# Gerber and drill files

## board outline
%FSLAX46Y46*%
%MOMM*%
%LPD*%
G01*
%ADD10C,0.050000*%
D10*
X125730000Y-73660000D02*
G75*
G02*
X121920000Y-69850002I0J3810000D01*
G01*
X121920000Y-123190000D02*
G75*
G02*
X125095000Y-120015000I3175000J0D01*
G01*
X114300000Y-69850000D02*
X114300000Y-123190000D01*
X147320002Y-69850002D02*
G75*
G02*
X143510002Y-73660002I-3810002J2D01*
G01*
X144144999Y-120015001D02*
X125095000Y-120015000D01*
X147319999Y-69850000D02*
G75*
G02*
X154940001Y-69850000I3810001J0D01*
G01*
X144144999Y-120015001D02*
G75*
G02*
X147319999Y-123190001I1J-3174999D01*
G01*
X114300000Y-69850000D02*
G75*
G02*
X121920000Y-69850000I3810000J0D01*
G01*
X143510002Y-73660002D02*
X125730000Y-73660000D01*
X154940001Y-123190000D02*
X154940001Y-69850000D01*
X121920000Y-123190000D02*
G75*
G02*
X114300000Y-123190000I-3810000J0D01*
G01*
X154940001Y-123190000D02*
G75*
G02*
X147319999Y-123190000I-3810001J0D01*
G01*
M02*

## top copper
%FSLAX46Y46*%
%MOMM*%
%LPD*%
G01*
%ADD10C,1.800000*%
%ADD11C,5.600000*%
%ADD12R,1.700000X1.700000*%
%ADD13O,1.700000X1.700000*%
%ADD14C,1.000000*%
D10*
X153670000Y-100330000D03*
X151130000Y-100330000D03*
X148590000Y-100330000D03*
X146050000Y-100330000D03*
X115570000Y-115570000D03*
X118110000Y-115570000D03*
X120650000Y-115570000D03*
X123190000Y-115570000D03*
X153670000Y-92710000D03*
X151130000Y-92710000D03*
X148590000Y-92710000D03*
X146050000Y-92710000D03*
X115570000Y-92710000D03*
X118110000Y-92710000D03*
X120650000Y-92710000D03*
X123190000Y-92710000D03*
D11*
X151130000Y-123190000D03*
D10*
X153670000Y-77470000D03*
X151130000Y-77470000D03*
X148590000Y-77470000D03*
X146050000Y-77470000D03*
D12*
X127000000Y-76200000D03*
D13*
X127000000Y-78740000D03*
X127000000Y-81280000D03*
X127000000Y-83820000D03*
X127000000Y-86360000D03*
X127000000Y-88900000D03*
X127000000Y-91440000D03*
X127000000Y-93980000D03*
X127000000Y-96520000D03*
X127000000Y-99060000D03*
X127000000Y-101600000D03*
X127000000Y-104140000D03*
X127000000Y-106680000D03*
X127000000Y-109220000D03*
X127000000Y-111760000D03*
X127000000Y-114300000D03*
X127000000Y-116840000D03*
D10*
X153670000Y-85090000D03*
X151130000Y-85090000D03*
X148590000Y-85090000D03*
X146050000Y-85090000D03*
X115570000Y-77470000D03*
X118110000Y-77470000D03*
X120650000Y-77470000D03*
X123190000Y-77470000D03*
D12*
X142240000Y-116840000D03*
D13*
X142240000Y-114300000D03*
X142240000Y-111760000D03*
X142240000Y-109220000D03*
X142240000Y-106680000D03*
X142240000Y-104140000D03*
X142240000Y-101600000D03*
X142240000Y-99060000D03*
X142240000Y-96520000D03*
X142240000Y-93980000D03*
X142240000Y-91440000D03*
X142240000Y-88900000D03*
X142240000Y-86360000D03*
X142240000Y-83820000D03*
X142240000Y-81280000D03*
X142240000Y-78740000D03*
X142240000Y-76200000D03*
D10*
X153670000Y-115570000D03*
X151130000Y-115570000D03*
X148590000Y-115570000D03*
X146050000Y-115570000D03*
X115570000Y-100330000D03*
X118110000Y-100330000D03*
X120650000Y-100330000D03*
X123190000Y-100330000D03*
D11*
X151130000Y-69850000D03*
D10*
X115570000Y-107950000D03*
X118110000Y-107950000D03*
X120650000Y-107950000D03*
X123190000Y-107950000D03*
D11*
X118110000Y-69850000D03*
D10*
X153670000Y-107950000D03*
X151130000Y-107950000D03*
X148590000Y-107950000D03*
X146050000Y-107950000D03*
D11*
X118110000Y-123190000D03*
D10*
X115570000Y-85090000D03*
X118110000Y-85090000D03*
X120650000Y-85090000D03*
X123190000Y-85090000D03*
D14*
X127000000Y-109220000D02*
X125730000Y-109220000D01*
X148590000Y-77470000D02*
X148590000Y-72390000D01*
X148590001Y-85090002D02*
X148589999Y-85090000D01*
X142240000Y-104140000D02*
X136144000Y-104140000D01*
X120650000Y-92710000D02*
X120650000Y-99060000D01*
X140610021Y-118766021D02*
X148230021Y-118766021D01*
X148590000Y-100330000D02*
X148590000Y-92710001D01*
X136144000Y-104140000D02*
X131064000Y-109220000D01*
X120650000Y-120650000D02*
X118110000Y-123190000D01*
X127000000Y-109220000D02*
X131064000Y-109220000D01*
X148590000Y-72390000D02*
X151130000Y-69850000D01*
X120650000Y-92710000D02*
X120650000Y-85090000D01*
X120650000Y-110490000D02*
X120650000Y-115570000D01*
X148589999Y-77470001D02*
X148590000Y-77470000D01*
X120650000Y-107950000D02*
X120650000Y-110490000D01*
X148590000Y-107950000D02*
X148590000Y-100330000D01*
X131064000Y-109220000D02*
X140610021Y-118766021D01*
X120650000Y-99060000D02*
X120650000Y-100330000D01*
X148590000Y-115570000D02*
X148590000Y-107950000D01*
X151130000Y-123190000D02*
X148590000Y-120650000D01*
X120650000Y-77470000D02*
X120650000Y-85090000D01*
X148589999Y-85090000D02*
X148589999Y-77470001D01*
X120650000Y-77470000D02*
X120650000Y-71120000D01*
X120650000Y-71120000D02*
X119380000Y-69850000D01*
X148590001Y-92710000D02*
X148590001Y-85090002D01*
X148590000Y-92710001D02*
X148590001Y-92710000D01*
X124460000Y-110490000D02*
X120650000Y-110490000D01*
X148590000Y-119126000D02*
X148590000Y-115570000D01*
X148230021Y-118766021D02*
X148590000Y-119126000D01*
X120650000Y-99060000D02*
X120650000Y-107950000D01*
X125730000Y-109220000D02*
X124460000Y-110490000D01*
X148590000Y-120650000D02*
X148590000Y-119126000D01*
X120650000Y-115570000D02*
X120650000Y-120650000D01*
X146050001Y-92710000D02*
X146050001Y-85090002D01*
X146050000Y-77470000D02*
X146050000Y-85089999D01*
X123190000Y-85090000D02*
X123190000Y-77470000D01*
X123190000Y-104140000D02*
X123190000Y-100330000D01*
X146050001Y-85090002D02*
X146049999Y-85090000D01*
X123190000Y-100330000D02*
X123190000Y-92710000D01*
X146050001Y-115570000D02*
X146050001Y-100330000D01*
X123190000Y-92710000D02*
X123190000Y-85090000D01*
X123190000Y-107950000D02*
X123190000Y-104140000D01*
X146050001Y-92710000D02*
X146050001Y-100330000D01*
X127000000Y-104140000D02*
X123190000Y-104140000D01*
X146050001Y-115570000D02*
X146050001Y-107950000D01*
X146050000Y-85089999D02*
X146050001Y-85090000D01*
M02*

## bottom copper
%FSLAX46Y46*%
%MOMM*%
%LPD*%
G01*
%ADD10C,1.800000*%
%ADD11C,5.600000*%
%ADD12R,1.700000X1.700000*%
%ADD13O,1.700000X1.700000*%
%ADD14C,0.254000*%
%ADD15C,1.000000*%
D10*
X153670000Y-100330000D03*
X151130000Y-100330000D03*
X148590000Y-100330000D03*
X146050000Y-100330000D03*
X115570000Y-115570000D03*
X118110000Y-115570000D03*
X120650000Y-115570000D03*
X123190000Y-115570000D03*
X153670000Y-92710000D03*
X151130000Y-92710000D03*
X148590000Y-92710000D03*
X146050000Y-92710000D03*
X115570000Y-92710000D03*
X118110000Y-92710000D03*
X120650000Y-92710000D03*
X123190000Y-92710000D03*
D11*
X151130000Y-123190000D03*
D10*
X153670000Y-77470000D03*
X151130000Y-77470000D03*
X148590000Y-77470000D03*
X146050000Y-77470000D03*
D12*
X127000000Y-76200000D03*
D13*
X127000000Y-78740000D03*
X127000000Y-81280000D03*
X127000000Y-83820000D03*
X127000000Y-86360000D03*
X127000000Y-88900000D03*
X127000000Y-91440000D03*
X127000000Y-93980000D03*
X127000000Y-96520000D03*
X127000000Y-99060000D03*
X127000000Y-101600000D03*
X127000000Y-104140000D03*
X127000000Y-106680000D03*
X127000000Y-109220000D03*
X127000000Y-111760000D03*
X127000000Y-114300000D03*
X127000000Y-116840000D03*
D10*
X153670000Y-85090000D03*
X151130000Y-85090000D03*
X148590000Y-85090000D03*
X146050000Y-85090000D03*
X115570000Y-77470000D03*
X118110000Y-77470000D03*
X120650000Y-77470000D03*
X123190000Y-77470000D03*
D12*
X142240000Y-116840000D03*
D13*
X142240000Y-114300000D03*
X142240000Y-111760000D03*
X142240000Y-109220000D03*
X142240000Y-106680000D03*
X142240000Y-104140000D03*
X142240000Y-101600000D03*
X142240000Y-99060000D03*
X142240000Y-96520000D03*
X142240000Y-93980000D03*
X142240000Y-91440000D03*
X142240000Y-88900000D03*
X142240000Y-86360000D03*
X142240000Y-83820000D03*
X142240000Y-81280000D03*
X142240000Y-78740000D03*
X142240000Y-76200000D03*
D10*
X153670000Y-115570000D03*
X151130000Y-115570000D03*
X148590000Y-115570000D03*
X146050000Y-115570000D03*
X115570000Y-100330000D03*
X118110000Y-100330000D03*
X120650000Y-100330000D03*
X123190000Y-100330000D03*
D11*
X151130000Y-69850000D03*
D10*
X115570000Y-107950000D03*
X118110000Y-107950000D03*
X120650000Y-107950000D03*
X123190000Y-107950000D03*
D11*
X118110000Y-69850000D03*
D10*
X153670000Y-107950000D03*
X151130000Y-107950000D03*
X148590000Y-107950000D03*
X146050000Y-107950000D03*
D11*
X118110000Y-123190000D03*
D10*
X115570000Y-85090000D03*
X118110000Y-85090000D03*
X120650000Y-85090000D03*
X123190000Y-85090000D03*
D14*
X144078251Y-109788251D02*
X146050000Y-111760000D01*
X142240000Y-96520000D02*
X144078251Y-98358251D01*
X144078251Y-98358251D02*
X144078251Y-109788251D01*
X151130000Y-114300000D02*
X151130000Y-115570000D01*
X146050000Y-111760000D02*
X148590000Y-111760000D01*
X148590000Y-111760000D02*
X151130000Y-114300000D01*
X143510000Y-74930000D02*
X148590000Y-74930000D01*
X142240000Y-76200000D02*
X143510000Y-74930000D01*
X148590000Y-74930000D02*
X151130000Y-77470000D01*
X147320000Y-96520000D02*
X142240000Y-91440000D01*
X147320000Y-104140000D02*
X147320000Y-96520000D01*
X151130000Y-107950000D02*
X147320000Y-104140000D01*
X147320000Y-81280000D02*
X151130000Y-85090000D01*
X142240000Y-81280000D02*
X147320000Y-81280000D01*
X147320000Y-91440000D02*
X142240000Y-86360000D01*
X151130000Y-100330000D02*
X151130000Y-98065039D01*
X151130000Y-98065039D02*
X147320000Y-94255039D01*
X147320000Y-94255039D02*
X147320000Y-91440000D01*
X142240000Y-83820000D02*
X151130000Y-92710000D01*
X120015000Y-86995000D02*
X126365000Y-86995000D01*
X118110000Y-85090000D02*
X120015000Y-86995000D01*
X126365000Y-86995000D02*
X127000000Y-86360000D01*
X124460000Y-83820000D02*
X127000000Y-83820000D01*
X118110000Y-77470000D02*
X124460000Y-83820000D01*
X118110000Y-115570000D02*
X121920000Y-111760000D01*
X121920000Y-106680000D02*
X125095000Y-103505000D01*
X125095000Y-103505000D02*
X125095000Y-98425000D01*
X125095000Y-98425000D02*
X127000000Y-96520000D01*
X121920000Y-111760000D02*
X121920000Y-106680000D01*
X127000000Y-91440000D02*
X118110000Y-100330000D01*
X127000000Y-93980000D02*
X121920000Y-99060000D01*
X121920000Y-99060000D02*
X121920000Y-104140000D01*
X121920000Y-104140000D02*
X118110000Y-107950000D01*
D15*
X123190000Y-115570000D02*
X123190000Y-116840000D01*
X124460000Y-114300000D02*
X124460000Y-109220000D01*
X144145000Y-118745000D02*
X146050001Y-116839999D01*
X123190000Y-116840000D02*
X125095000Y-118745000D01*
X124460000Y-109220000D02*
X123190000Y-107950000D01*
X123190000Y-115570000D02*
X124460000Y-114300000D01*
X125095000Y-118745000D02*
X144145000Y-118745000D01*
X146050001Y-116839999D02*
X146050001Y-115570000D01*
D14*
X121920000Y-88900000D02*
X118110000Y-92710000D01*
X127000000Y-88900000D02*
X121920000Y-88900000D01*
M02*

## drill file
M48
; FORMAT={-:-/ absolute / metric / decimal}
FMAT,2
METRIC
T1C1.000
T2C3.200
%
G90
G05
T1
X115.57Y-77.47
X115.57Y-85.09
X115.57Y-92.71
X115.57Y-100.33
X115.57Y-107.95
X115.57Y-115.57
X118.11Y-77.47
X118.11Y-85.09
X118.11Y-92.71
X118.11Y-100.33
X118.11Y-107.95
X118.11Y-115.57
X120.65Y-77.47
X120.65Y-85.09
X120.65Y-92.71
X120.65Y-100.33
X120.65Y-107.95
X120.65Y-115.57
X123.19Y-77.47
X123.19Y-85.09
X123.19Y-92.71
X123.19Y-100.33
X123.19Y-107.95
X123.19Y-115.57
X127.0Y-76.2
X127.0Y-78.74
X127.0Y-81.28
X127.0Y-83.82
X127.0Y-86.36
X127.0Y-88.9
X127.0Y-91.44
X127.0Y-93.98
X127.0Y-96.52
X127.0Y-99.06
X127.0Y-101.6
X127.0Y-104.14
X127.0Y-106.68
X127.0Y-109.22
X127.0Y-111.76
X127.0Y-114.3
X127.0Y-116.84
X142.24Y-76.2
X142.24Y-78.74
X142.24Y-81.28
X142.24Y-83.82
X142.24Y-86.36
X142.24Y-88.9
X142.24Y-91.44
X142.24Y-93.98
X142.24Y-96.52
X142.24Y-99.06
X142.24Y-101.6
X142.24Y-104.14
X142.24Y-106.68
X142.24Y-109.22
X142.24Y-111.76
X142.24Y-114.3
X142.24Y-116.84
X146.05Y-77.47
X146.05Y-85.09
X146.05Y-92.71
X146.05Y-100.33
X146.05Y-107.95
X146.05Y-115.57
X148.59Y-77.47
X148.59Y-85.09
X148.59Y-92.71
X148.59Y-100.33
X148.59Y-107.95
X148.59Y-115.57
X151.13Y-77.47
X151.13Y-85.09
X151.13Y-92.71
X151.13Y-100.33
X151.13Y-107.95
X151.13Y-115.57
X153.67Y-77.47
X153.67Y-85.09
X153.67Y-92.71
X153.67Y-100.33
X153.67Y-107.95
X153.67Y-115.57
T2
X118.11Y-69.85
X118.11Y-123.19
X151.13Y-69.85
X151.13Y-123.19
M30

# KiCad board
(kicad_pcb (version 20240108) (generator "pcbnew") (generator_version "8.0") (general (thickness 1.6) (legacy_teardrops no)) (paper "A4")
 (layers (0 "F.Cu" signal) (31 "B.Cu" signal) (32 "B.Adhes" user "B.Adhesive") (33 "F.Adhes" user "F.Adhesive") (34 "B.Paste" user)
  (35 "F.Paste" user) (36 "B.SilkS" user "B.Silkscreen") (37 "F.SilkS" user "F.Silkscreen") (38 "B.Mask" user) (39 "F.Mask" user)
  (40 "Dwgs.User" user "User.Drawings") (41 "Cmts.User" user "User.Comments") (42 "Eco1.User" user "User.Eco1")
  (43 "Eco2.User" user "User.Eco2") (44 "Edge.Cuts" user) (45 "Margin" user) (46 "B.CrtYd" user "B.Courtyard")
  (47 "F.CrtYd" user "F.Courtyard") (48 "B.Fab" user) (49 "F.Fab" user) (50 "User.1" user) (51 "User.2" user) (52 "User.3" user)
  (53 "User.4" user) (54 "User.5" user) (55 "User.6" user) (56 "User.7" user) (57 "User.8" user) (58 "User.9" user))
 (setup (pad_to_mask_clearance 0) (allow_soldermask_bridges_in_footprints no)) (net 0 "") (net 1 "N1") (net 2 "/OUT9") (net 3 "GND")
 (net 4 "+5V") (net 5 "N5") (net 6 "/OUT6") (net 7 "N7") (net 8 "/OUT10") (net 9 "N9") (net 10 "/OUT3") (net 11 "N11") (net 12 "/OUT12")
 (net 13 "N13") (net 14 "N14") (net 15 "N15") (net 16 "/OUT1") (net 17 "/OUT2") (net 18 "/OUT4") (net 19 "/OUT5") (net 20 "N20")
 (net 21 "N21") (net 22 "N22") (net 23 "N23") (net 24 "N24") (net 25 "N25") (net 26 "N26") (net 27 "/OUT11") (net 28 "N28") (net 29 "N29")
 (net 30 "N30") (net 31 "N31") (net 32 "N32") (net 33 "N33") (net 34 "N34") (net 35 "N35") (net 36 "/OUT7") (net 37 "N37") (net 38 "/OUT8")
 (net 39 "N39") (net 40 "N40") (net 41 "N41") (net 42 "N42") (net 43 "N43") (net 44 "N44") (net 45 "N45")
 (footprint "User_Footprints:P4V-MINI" (layer "F.Cu") (at 153.67 100.33 180)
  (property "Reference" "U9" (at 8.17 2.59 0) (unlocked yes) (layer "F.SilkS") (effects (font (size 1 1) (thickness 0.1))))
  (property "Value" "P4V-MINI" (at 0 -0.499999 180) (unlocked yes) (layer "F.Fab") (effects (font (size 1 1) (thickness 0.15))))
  (pad "1" thru_hole circle (at 0 0 180) (size 1.8 1.8) (drill 1) (layers "*.Cu" "*.Mask") (remove_unused_layers no) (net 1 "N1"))
  (pad "2" thru_hole circle (at 2.54 0 180) (size 1.8 1.8) (drill 1) (layers "*.Cu" "*.Mask") (remove_unused_layers no) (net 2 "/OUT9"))
  (pad "3" thru_hole circle (at 5.08 0 180) (size 1.8 1.8) (drill 1) (layers "*.Cu" "*.Mask") (remove_unused_layers no) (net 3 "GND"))
  (pad "4" thru_hole circle (at 7.62 0 180) (size 1.8 1.8) (drill 1) (layers "*.Cu" "*.Mask") (remove_unused_layers no) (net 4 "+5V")))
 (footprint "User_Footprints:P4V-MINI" (layer "F.Cu") (at 115.57 115.57)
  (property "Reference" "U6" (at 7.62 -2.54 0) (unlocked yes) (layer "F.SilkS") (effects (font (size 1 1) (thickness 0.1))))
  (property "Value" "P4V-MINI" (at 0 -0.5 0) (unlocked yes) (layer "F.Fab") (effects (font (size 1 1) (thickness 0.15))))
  (pad "1" thru_hole circle (at 0 0) (size 1.8 1.8) (drill 1) (layers "*.Cu" "*.Mask") (remove_unused_layers no) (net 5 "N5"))
  (pad "2" thru_hole circle (at 2.54 0) (size 1.8 1.8) (drill 1) (layers "*.Cu" "*.Mask") (remove_unused_layers no) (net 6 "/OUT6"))
  (pad "3" thru_hole circle (at 5.08 0) (size 1.8 1.8) (drill 1) (layers "*.Cu" "*.Mask") (remove_unused_layers no) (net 3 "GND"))
  (pad "4" thru_hole circle (at 7.62 0) (size 1.8 1.8) (drill 1) (layers "*.Cu" "*.Mask") (remove_unused_layers no) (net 4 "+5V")))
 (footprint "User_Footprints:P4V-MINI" (layer "F.Cu") (at 153.67 92.71 180)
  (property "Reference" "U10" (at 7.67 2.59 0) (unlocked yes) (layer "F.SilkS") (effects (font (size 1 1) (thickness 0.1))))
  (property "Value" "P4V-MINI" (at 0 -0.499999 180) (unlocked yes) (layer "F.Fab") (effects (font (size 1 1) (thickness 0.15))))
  (pad "1" thru_hole circle (at 0 0 180) (size 1.8 1.8) (drill 1) (layers "*.Cu" "*.Mask") (remove_unused_layers no) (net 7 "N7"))
  (pad "2" thru_hole circle (at 2.54 0 180) (size 1.8 1.8) (drill 1) (layers "*.Cu" "*.Mask") (remove_unused_layers no) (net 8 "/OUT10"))
  (pad "3" thru_hole circle (at 5.08 0 180) (size 1.8 1.8) (drill 1) (layers "*.Cu" "*.Mask") (remove_unused_layers no) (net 3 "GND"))
  (pad "4" thru_hole circle (at 7.62 0 180) (size 1.8 1.8) (drill 1) (layers "*.Cu" "*.Mask") (remove_unused_layers no) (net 4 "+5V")))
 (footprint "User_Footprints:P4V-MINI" (layer "F.Cu") (at 115.57 92.71)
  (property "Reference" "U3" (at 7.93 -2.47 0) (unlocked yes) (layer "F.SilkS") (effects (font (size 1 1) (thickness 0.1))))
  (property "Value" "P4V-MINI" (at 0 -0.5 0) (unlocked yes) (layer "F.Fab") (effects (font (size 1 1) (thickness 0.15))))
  (pad "1" thru_hole circle (at 0 0) (size 1.8 1.8) (drill 1) (layers "*.Cu" "*.Mask") (remove_unused_layers no) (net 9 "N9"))
  (pad "2" thru_hole circle (at 2.54 0) (size 1.8 1.8) (drill 1) (layers "*.Cu" "*.Mask") (remove_unused_layers no) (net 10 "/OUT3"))
  (pad "3" thru_hole circle (at 5.08 0) (size 1.8 1.8) (drill 1) (layers "*.Cu" "*.Mask") (remove_unused_layers no) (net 3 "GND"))
  (pad "4" thru_hole circle (at 7.62 0) (size 1.8 1.8) (drill 1) (layers "*.Cu" "*.Mask") (remove_unused_layers no) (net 4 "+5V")))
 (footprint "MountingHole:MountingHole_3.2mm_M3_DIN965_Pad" (layer "F.Cu") (at 151.13 123.19)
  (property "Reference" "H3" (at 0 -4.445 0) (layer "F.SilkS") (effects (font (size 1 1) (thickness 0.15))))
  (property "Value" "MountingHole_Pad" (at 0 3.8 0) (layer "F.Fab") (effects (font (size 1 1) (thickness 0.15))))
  (pad "1" thru_hole circle (at 0 0) (size 5.6 5.6) (drill 3.2) (layers "*.Cu" "*.Mask") (remove_unused_layers no) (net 3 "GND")))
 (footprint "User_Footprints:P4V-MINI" (layer "F.Cu") (at 153.67 77.47 180)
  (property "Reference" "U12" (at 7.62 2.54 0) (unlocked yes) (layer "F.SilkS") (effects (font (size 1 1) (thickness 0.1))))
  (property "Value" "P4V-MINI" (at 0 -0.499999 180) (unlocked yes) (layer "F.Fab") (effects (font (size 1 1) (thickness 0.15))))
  (pad "1" thru_hole circle (at 0 0 180) (size 1.8 1.8) (drill 1) (layers "*.Cu" "*.Mask") (remove_unused_layers no) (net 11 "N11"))
  (pad "2" thru_hole circle (at 2.54 0 180) (size 1.8 1.8) (drill 1) (layers "*.Cu" "*.Mask") (remove_unused_layers no) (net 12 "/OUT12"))
  (pad "3" thru_hole circle (at 5.08 0 180) (size 1.8 1.8) (drill 1) (layers "*.Cu" "*.Mask") (remove_unused_layers no) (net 3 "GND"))
  (pad "4" thru_hole circle (at 7.62 0 180) (size 1.8 1.8) (drill 1) (layers "*.Cu" "*.Mask") (remove_unused_layers no) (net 4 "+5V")))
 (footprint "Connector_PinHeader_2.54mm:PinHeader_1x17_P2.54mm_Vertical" (layer "F.Cu") (at 127 76.2)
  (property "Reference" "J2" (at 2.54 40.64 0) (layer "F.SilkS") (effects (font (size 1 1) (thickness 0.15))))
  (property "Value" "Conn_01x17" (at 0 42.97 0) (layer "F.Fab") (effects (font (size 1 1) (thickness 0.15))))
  (pad "1" thru_hole rect (at 0 0) (size 1.7 1.7) (drill 1) (layers "*.Cu" "*.Mask") (remove_unused_layers no) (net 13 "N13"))
  (pad "2" thru_hole oval (at 0 2.54) (size 1.7 1.7) (drill 1) (layers "*.Cu" "*.Mask") (remove_unused_layers no) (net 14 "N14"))
  (pad "3" thru_hole oval (at 0 5.08) (size 1.7 1.7) (drill 1) (layers "*.Cu" "*.Mask") (remove_unused_layers no) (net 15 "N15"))
  (pad "4" thru_hole oval (at 0 7.62) (size 1.7 1.7) (drill 1) (layers "*.Cu" "*.Mask") (remove_unused_layers no) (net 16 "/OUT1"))
  (pad "5" thru_hole oval (at 0 10.16) (size 1.7 1.7) (drill 1) (layers "*.Cu" "*.Mask") (remove_unused_layers no) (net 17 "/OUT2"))
  (pad "6" thru_hole oval (at 0 12.7) (size 1.7 1.7) (drill 1) (layers "*.Cu" "*.Mask") (remove_unused_layers no) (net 10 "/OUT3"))
  (pad "7" thru_hole oval (at 0 15.24) (size 1.7 1.7) (drill 1) (layers "*.Cu" "*.Mask") (remove_unused_layers no) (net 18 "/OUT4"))
  (pad "8" thru_hole oval (at 0 17.78) (size 1.7 1.7) (drill 1) (layers "*.Cu" "*.Mask") (remove_unused_layers no) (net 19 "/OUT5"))
  (pad "9" thru_hole oval (at 0 20.32) (size 1.7 1.7) (drill 1) (layers "*.Cu" "*.Mask") (remove_unused_layers no) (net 6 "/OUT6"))
  (pad "10" thru_hole oval (at 0 22.86) (size 1.7 1.7) (drill 1) (layers "*.Cu" "*.Mask") (remove_unused_layers no) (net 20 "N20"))
  (pad "11" thru_hole oval (at 0 25.4) (size 1.7 1.7) (drill 1) (layers "*.Cu" "*.Mask") (remove_unused_layers no) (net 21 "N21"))
  (pad "12" thru_hole oval (at 0 27.94) (size 1.7 1.7) (drill 1) (layers "*.Cu" "*.Mask") (remove_unused_layers no) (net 4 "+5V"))
  (pad "13" thru_hole oval (at 0 30.48) (size 1.7 1.7) (drill 1) (layers "*.Cu" "*.Mask") (remove_unused_layers no) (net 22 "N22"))
  (pad "14" thru_hole oval (at 0 33.02) (size 1.7 1.7) (drill 1) (layers "*.Cu" "*.Mask") (remove_unused_layers no) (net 3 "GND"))
  (pad "15" thru_hole oval (at 0 35.56) (size 1.7 1.7) (drill 1) (layers "*.Cu" "*.Mask") (remove_unused_layers no) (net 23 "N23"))
  (pad "16" thru_hole oval (at 0 38.1) (size 1.7 1.7) (drill 1) (layers "*.Cu" "*.Mask") (remove_unused_layers no) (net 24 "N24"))
  (pad "17" thru_hole oval (at 0 40.64) (size 1.7 1.7) (drill 1) (layers "*.Cu" "*.Mask") (remove_unused_layers no) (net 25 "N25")))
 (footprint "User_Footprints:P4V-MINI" (layer "F.Cu") (at 153.67 85.09 180)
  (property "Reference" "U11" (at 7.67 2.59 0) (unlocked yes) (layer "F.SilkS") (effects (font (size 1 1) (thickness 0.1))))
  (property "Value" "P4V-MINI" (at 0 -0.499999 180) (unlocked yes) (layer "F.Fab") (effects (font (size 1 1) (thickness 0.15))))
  (pad "1" thru_hole circle (at 0 0 180) (size 1.8 1.8) (drill 1) (layers "*.Cu" "*.Mask") (remove_unused_layers no) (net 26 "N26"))
  (pad "2" thru_hole circle (at 2.54 0 180) (size 1.8 1.8) (drill 1) (layers "*.Cu" "*.Mask") (remove_unused_layers no) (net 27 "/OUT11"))
  (pad "3" thru_hole circle (at 5.08 0 180) (size 1.8 1.8) (drill 1) (layers "*.Cu" "*.Mask") (remove_unused_layers no) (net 3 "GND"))
  (pad "4" thru_hole circle (at 7.62 0 180) (size 1.8 1.8) (drill 1) (layers "*.Cu" "*.Mask") (remove_unused_layers no) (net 4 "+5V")))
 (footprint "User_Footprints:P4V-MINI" (layer "F.Cu") (at 115.57 77.47)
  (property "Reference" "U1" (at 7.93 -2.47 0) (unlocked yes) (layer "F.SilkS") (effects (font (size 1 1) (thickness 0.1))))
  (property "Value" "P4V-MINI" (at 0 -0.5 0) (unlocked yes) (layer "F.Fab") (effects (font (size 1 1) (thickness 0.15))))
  (pad "1" thru_hole circle (at 0 0) (size 1.8 1.8) (drill 1) (layers "*.Cu" "*.Mask") (remove_unused_layers no) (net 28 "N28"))
  (pad "2" thru_hole circle (at 2.54 0) (size 1.8 1.8) (drill 1) (layers "*.Cu" "*.Mask") (remove_unused_layers no) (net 16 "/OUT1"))
  (pad "3" thru_hole circle (at 5.08 0) (size 1.8 1.8) (drill 1) (layers "*.Cu" "*.Mask") (remove_unused_layers no) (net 3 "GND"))
  (pad "4" thru_hole circle (at 7.62 0) (size 1.8 1.8) (drill 1) (layers "*.Cu" "*.Mask") (remove_unused_layers no) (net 4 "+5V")))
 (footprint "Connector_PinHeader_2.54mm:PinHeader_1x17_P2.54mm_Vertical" (layer "F.Cu") (at 142.24 116.84 180)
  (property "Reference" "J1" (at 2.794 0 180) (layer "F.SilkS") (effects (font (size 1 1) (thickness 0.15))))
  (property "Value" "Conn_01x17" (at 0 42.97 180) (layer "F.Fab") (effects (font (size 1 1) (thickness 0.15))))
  (pad "1" thru_hole rect (at 0 0 180) (size 1.7 1.7) (drill 1) (layers "*.Cu" "*.Mask") (remove_unused_layers no) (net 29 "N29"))
  (pad "2" thru_hole oval (at 0 2.54 180) (size 1.7 1.7) (drill 1) (layers "*.Cu" "*.Mask") (remove_unused_layers no) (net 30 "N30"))
  (pad "3" thru_hole oval (at 0 5.08 180) (size 1.7 1.7) (drill 1) (layers "*.Cu" "*.Mask") (remove_unused_layers no) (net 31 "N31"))
  (pad "4" thru_hole oval (at 0 7.62 180) (size 1.7 1.7) (drill 1) (layers "*.Cu" "*.Mask") (remove_unused_layers no) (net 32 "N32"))
  (pad "5" thru_hole oval (at 0 10.16 180) (size 1.7 1.7) (drill 1) (layers "*.Cu" "*.Mask") (remove_unused_layers no) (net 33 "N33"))
  (pad "6" thru_hole oval (at 0 12.7 180) (size 1.7 1.7) (drill 1) (layers "*.Cu" "*.Mask") (remove_unused_layers no) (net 3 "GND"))
  (pad "7" thru_hole oval (at 0 15.24 180) (size 1.7 1.7) (drill 1) (layers "*.Cu" "*.Mask") (remove_unused_layers no) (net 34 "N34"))
  (pad "8" thru_hole oval (at 0 17.78 180) (size 1.7 1.7) (drill 1) (layers "*.Cu" "*.Mask") (remove_unused_layers no) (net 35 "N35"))
  (pad "9" thru_hole oval (at 0 20.32 180) (size 1.7 1.7) (drill 1) (layers "*.Cu" "*.Mask") (remove_unused_layers no) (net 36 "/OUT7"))
  (pad "10" thru_hole oval (at 0 22.86 180) (size 1.7 1.7) (drill 1) (layers "*.Cu" "*.Mask") (remove_unused_layers no) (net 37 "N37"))
  (pad "11" thru_hole oval (at 0 25.4 180) (size 1.7 1.7) (drill 1) (layers "*.Cu" "*.Mask") (remove_unused_layers no) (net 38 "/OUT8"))
  (pad "12" thru_hole oval (at 0 27.94 180) (size 1.7 1.7) (drill 1) (layers "*.Cu" "*.Mask") (remove_unused_layers no) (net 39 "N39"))
  (pad "13" thru_hole oval (at 0 30.48 180) (size 1.7 1.7) (drill 1) (layers "*.Cu" "*.Mask") (remove_unused_layers no) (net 2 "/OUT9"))
  (pad "14" thru_hole oval (at 0 33.02 180) (size 1.7 1.7) (drill 1) (layers "*.Cu" "*.Mask") (remove_unused_layers no) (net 8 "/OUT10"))
  (pad "15" thru_hole oval (at 0 35.56 180) (size 1.7 1.7) (drill 1) (layers "*.Cu" "*.Mask") (remove_unused_layers no) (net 27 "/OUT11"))
  (pad "16" thru_hole oval (at 0 38.1 180) (size 1.7 1.7) (drill 1) (layers "*.Cu" "*.Mask") (remove_unused_layers no) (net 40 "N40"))
  (pad "17" thru_hole oval (at 0 40.64 180) (size 1.7 1.7) (drill 1) (layers "*.Cu" "*.Mask") (remove_unused_layers no) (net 12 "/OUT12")))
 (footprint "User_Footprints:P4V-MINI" (layer "F.Cu") (at 153.67 115.57 180)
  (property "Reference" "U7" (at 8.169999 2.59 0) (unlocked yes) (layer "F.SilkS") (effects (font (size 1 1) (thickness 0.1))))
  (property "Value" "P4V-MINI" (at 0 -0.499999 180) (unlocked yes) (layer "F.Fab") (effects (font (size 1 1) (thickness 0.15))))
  (pad "1" thru_hole circle (at 0 0 180) (size 1.8 1.8) (drill 1) (layers "*.Cu" "*.Mask") (remove_unused_layers no) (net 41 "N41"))
  (pad "2" thru_hole circle (at 2.54 0 180) (size 1.8 1.8) (drill 1) (layers "*.Cu" "*.Mask") (remove_unused_layers no) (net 36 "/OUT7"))
  (pad "3" thru_hole circle (at 5.08 0 180) (size 1.8 1.8) (drill 1) (layers "*.Cu" "*.Mask") (remove_unused_layers no) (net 3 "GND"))
  (pad "4" thru_hole circle (at 7.62 0 180) (size 1.8 1.8) (drill 1) (layers "*.Cu" "*.Mask") (remove_unused_layers no) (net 4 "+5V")))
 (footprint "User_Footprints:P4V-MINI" (layer "F.Cu") (at 115.57 100.33)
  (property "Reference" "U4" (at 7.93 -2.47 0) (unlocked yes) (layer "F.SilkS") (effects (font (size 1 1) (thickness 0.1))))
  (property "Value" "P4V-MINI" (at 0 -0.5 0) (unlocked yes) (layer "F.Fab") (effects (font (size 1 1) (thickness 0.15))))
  (pad "1" thru_hole circle (at 0 0) (size 1.8 1.8) (drill 1) (layers "*.Cu" "*.Mask") (remove_unused_layers no) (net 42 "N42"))
  (pad "2" thru_hole circle (at 2.54 0) (size 1.8 1.8) (drill 1) (layers "*.Cu" "*.Mask") (remove_unused_layers no) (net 18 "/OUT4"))
  (pad "3" thru_hole circle (at 5.08 0) (size 1.8 1.8) (drill 1) (layers "*.Cu" "*.Mask") (remove_unused_layers no) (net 3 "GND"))
  (pad "4" thru_hole circle (at 7.62 0) (size 1.8 1.8) (drill 1) (layers "*.Cu" "*.Mask") (remove_unused_layers no) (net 4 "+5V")))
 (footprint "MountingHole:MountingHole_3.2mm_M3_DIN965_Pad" (layer "F.Cu") (at 151.13 69.85)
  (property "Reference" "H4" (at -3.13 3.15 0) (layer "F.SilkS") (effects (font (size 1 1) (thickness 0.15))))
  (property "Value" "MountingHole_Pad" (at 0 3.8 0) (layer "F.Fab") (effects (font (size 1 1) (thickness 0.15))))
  (pad "1" thru_hole circle (at 0 0) (size 5.6 5.6) (drill 3.2) (layers "*.Cu" "*.Mask") (remove_unused_layers no) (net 3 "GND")))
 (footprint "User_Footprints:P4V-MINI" (layer "F.Cu") (at 115.57 107.95)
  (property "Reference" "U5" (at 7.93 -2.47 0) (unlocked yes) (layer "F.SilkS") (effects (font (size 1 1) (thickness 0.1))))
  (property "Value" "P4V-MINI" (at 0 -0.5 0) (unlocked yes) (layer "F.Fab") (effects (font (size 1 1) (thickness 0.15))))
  (pad "1" thru_hole circle (at 0 0) (size 1.8 1.8) (drill 1) (layers "*.Cu" "*.Mask") (remove_unused_layers no) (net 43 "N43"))
  (pad "2" thru_hole circle (at 2.54 0) (size 1.8 1.8) (drill 1) (layers "*.Cu" "*.Mask") (remove_unused_layers no) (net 19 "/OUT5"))
  (pad "3" thru_hole circle (at 5.08 0) (size 1.8 1.8) (drill 1) (layers "*.Cu" "*.Mask") (remove_unused_layers no) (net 3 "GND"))
  (pad "4" thru_hole circle (at 7.62 0) (size 1.8 1.8) (drill 1) (layers "*.Cu" "*.Mask") (remove_unused_layers no) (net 4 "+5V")))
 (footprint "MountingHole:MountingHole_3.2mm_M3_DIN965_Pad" (layer "F.Cu") (at 118.11 69.85)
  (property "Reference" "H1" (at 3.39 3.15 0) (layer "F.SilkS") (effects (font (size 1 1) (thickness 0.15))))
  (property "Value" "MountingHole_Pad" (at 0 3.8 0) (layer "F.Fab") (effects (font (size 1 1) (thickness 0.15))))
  (pad "1" thru_hole circle (at 0 0) (size 5.6 5.6) (drill 3.2) (layers "*.Cu" "*.Mask") (remove_unused_layers no) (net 3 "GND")))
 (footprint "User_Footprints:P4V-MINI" (layer "F.Cu") (at 153.67 107.95 180)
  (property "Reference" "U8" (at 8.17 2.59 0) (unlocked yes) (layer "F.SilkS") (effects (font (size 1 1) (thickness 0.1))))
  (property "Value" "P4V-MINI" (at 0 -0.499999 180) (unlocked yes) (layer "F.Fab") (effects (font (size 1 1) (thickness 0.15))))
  (pad "1" thru_hole circle (at 0 0 180) (size 1.8 1.8) (drill 1) (layers "*.Cu" "*.Mask") (remove_unused_layers no) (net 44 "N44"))
  (pad "2" thru_hole circle (at 2.54 0 180) (size 1.8 1.8) (drill 1) (layers "*.Cu" "*.Mask") (remove_unused_layers no) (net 38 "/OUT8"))
  (pad "3" thru_hole circle (at 5.08 0 180) (size 1.8 1.8) (drill 1) (layers "*.Cu" "*.Mask") (remove_unused_layers no) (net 3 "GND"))
  (pad "4" thru_hole circle (at 7.62 0 180) (size 1.8 1.8) (drill 1) (layers "*.Cu" "*.Mask") (remove_unused_layers no) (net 4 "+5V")))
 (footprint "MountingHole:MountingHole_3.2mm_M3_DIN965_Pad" (layer "F.Cu") (at 118.11 123.19)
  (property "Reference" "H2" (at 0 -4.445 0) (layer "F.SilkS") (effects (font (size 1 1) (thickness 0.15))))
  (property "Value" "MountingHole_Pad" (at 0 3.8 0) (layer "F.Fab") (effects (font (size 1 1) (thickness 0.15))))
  (pad "1" thru_hole circle (at 0 0) (size 5.6 5.6) (drill 3.2) (layers "*.Cu" "*.Mask") (remove_unused_layers no) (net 3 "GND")))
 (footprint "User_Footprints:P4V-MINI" (layer "F.Cu") (at 115.57 85.09)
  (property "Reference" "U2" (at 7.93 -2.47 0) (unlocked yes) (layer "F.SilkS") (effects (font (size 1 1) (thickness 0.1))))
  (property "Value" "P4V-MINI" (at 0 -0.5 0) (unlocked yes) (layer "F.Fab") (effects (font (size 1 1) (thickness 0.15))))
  (pad "1" thru_hole circle (at 0 0) (size 1.8 1.8) (drill 1) (layers "*.Cu" "*.Mask") (remove_unused_layers no) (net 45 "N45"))
  (pad "2" thru_hole circle (at 2.54 0) (size 1.8 1.8) (drill 1) (layers "*.Cu" "*.Mask") (remove_unused_layers no) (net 17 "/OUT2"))
  (pad "3" thru_hole circle (at 5.08 0) (size 1.8 1.8) (drill 1) (layers "*.Cu" "*.Mask") (remove_unused_layers no) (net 3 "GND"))
  (pad "4" thru_hole circle (at 7.62 0) (size 1.8 1.8) (drill 1) (layers "*.Cu" "*.Mask") (remove_unused_layers no) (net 4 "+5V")))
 (gr_arc (start 125.73 73.66) (mid 123.035924 72.544078) (end 121.92 69.850002) (stroke (width 0.05) (type default)) (layer "Edge.Cuts"))
 (gr_arc (start 121.92 123.19) (mid 122.849936 120.944936) (end 125.095 120.015) (stroke (width 0.05) (type default)) (layer "Edge.Cuts"))
 (gr_line (start 114.3 69.85) (end 114.3 123.19) (stroke (width 0.05) (type default)) (layer "Edge.Cuts"))
 (gr_arc (start 147.320002 69.850002) (mid 146.204078 72.544078) (end 143.510002 73.660002) (stroke (width 0.05) (type default))
  (layer "Edge.Cuts"))
 (gr_line (start 144.144999 120.015001) (end 125.095 120.015) (stroke (width 0.05) (type default)) (layer "Edge.Cuts"))
 (gr_arc (start 147.319999 69.85) (mid 151.13 66.039999) (end 154.940001 69.85) (stroke (width 0.05) (type default)) (layer "Edge.Cuts"))
 (gr_arc (start 144.144999 120.015001) (mid 146.390063 120.944937) (end 147.319999 123.190001) (stroke (width 0.05) (type default))
  (layer "Edge.Cuts"))
 (gr_arc (start 114.3 69.85) (mid 118.11 66.04) (end 121.92 69.85) (stroke (width 0.05) (type default)) (layer "Edge.Cuts"))
 (gr_line (start 143.510002 73.660002) (end 125.73 73.66) (stroke (width 0.05) (type default)) (layer "Edge.Cuts"))
 (gr_line (start 154.940001 123.19) (end 154.940001 69.85) (stroke (width 0.05) (type default)) (layer "Edge.Cuts"))
 (gr_arc (start 121.92 123.19) (mid 118.11 127) (end 114.3 123.19) (stroke (width 0.05) (type default)) (layer "Edge.Cuts"))
 (gr_arc (start 154.940001 123.19) (mid 151.13 127.000001) (end 147.319999 123.19) (stroke (width 0.05) (type default)) (layer "Edge.Cuts"))
 (segment (start 144.078251 109.788251) (end 146.05 111.76) (width 0.254) (layer "B.Cu") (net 36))
 (segment (start 142.24 96.52) (end 144.078251 98.358251) (width 0.254) (layer "B.Cu") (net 36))
 (segment (start 144.078251 98.358251) (end 144.078251 109.788251) (width 0.254) (layer "B.Cu") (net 36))
 (segment (start 151.13 114.3) (end 151.13 115.57) (width 0.254) (layer "B.Cu") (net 36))
 (segment (start 146.05 111.76) (end 148.59 111.76) (width 0.254) (layer "B.Cu") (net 36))
 (segment (start 148.59 111.76) (end 151.13 114.3) (width 0.254) (layer "B.Cu") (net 36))
 (segment (start 143.51 74.93) (end 148.59 74.93) (width 0.254) (layer "B.Cu") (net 12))
 (segment (start 142.24 76.2) (end 143.51 74.93) (width 0.254) (layer "B.Cu") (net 12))
 (segment (start 148.59 74.93) (end 151.13 77.47) (width 0.254) (layer "B.Cu") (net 12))
 (segment (start 147.32 96.52) (end 142.24 91.44) (width 0.254) (layer "B.Cu") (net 38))
 (segment (start 147.32 104.14) (end 147.32 96.52) (width 0.254) (layer "B.Cu") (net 38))
 (segment (start 151.13 107.95) (end 147.32 104.14) (width 0.254) (layer "B.Cu") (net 38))
 (segment (start 147.32 81.28) (end 151.13 85.09) (width 0.254) (layer "B.Cu") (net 27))
 (segment (start 142.24 81.28) (end 147.32 81.28) (width 0.254) (layer "B.Cu") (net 27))
 (segment (start 147.32 91.44) (end 142.24 86.36) (width 0.254) (layer "B.Cu") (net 2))
 (segment (start 151.13 100.33) (end 151.13 98.065039) (width 0.254) (layer "B.Cu") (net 2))
 (segment (start 151.13 98.065039) (end 147.32 94.255039) (width 0.254) (layer "B.Cu") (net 2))
 (segment (start 147.32 94.255039) (end 147.32 91.44) (width 0.254) (layer "B.Cu") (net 2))
 (segment (start 127 109.22) (end 125.73 109.22) (width 1) (layer "F.Cu") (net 3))
 (segment (start 148.59 77.47) (end 148.59 72.39) (width 1) (layer "F.Cu") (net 3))
 (segment (start 148.590001 85.090002) (end 148.589999 85.09) (width 1) (layer "F.Cu") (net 3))
 (segment (start 142.24 104.14) (end 136.144 104.14) (width 1) (layer "F.Cu") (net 3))
 (segment (start 120.65 92.71) (end 120.65 99.06) (width 1) (layer "F.Cu") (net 3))
 (segment (start 140.610021 118.766021) (end 148.230021 118.766021) (width 1) (layer "F.Cu") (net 3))
 (segment (start 148.59 100.33) (end 148.59 92.710001) (width 1) (layer "F.Cu") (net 3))
 (segment (start 136.144 104.14) (end 131.064 109.22) (width 1) (layer "F.Cu") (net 3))
 (segment (start 120.65 120.65) (end 118.11 123.19) (width 1) (layer "F.Cu") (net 3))
 (segment (start 127 109.22) (end 131.064 109.22) (width 1) (layer "F.Cu") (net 3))
 (segment (start 148.59 72.39) (end 151.13 69.85) (width 1) (layer "F.Cu") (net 3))
 (segment (start 120.65 92.71) (end 120.65 85.09) (width 1) (layer "F.Cu") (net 3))
 (segment (start 120.65 110.49) (end 120.65 115.57) (width 1) (layer "F.Cu") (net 3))
 (segment (start 148.589999 77.470001) (end 148.59 77.47) (width 1) (layer "F.Cu") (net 3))
 (segment (start 120.65 107.95) (end 120.65 110.49) (width 1) (layer "F.Cu") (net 3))
 (segment (start 148.59 107.95) (end 148.59 100.33) (width 1) (layer "F.Cu") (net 3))
 (segment (start 131.064 109.22) (end 140.610021 118.766021) (width 1) (layer "F.Cu") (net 3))
 (segment (start 120.65 99.06) (end 120.65 100.33) (width 1) (layer "F.Cu") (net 3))
 (segment (start 148.59 115.57) (end 148.59 107.95) (width 1) (layer "F.Cu") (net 3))
 (segment (start 151.13 123.19) (end 148.59 120.65) (width 1) (layer "F.Cu") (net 3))
 (segment (start 120.65 77.47) (end 120.65 85.09) (width 1) (layer "F.Cu") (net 3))
 (segment (start 148.589999 85.09) (end 148.589999 77.470001) (width 1) (layer "F.Cu") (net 3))
 (segment (start 120.65 77.47) (end 120.65 71.12) (width 1) (layer "F.Cu") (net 3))
 (segment (start 120.65 71.12) (end 119.38 69.85) (width 1) (layer "F.Cu") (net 3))
 (segment (start 148.590001 92.71) (end 148.590001 85.090002) (width 1) (layer "F.Cu") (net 3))
 (segment (start 148.59 92.710001) (end 148.590001 92.71) (width 1) (layer "F.Cu") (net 3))
 (segment (start 124.46 110.49) (end 120.65 110.49) (width 1) (layer "F.Cu") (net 3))
 (segment (start 148.59 119.126) (end 148.59 115.57) (width 1) (layer "F.Cu") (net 3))
 (segment (start 148.230021 118.766021) (end 148.59 119.126) (width 1) (layer "F.Cu") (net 3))
 (segment (start 120.65 99.06) (end 120.65 107.95) (width 1) (layer "F.Cu") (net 3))
 (segment (start 125.73 109.22) (end 124.46 110.49) (width 1) (layer "F.Cu") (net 3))
 (segment (start 148.59 120.65) (end 148.59 119.126) (width 1) (layer "F.Cu") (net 3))
 (segment (start 120.65 115.57) (end 120.65 120.65) (width 1) (layer "F.Cu") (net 3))
 (segment (start 142.24 83.82) (end 151.13 92.71) (width 0.254) (layer "B.Cu") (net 8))
 (segment (start 120.015 86.995) (end 126.365 86.995) (width 0.254) (layer "B.Cu") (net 17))
 (segment (start 118.11 85.09) (end 120.015 86.995) (width 0.254) (layer "B.Cu") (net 17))
 (segment (start 126.365 86.995) (end 127 86.36) (width 0.254) (layer "B.Cu") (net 17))
 (segment (start 124.46 83.82) (end 127 83.82) (width 0.254) (layer "B.Cu") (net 16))
 (segment (start 118.11 77.47) (end 124.46 83.82) (width 0.254) (layer "B.Cu") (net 16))
 (segment (start 118.11 115.57) (end 121.92 111.76) (width 0.254) (layer "B.Cu") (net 6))
 (segment (start 121.92 106.68) (end 125.095 103.505) (width 0.254) (layer "B.Cu") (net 6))
 (segment (start 125.095 103.505) (end 125.095 98.425) (width 0.254) (layer "B.Cu") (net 6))
 (segment (start 125.095 98.425) (end 127 96.52) (width 0.254) (layer "B.Cu") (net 6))
 (segment (start 121.92 111.76) (end 121.92 106.68) (width 0.254) (layer "B.Cu") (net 6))
 (segment (start 127 91.44) (end 118.11 100.33) (width 0.254) (layer "B.Cu") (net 18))
 (segment (start 127 93.98) (end 121.92 99.06) (width 0.254) (layer "B.Cu") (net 19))
 (segment (start 121.92 99.06) (end 121.92 104.14) (width 0.254) (layer "B.Cu") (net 19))
 (segment (start 121.92 104.14) (end 118.11 107.95) (width 0.254) (layer "B.Cu") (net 19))
 (segment (start 146.050001 92.71) (end 146.050001 85.090002) (width 1) (layer "F.Cu") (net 4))
 (segment (start 146.05 77.47) (end 146.05 85.089999) (width 1) (layer "F.Cu") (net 4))
 (segment (start 123.19 85.09) (end 123.19 77.47) (width 1) (layer "F.Cu") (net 4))
 (segment (start 123.19 104.14) (end 123.19 100.33) (width 1) (layer "F.Cu") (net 4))
 (segment (start 146.050001 85.090002) (end 146.049999 85.09) (width 1) (layer "F.Cu") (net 4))
 (segment (start 123.19 100.33) (end 123.19 92.71) (width 1) (layer "F.Cu") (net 4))
 (segment (start 146.050001 115.57) (end 146.050001 100.33) (width 1) (layer "F.Cu") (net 4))
 (segment (start 123.19 92.71) (end 123.19 85.09) (width 1) (layer "F.Cu") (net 4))
 (segment (start 123.19 107.95) (end 123.19 104.14) (width 1) (layer "F.Cu") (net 4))
 (segment (start 146.050001 92.71) (end 146.050001 100.33) (width 1) (layer "F.Cu") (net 4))
 (segment (start 127 104.14) (end 123.19 104.14) (width 1) (layer "F.Cu") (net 4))
 (segment (start 146.050001 115.57) (end 146.050001 107.95) (width 1) (layer "F.Cu") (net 4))
 (segment (start 146.05 85.089999) (end 146.050001 85.09) (width 1) (layer "F.Cu") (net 4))
 (segment (start 123.19 115.57) (end 123.19 116.84) (width 1) (layer "B.Cu") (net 4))
 (segment (start 124.46 114.3) (end 124.46 109.22) (width 1) (layer "B.Cu") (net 4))
 (segment (start 144.145 118.745) (end 146.050001 116.839999) (width 1) (layer "B.Cu") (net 4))
 (segment (start 123.19 116.84) (end 125.095 118.745) (width 1) (layer "B.Cu") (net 4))
 (segment (start 124.46 109.22) (end 123.19 107.95) (width 1) (layer "B.Cu") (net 4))
 (segment (start 123.19 115.57) (end 124.46 114.3) (width 1) (layer "B.Cu") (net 4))
 (segment (start 125.095 118.745) (end 144.145 118.745) (width 1) (layer "B.Cu") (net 4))
 (segment (start 146.050001 116.839999) (end 146.050001 115.57) (width 1) (layer "B.Cu") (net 4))
 (segment (start 121.92 88.9) (end 118.11 92.71) (width 0.254) (layer "B.Cu") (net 10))
 (segment (start 127 88.9) (end 121.92 88.9) (width 0.254) (layer "B.Cu") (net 10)))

